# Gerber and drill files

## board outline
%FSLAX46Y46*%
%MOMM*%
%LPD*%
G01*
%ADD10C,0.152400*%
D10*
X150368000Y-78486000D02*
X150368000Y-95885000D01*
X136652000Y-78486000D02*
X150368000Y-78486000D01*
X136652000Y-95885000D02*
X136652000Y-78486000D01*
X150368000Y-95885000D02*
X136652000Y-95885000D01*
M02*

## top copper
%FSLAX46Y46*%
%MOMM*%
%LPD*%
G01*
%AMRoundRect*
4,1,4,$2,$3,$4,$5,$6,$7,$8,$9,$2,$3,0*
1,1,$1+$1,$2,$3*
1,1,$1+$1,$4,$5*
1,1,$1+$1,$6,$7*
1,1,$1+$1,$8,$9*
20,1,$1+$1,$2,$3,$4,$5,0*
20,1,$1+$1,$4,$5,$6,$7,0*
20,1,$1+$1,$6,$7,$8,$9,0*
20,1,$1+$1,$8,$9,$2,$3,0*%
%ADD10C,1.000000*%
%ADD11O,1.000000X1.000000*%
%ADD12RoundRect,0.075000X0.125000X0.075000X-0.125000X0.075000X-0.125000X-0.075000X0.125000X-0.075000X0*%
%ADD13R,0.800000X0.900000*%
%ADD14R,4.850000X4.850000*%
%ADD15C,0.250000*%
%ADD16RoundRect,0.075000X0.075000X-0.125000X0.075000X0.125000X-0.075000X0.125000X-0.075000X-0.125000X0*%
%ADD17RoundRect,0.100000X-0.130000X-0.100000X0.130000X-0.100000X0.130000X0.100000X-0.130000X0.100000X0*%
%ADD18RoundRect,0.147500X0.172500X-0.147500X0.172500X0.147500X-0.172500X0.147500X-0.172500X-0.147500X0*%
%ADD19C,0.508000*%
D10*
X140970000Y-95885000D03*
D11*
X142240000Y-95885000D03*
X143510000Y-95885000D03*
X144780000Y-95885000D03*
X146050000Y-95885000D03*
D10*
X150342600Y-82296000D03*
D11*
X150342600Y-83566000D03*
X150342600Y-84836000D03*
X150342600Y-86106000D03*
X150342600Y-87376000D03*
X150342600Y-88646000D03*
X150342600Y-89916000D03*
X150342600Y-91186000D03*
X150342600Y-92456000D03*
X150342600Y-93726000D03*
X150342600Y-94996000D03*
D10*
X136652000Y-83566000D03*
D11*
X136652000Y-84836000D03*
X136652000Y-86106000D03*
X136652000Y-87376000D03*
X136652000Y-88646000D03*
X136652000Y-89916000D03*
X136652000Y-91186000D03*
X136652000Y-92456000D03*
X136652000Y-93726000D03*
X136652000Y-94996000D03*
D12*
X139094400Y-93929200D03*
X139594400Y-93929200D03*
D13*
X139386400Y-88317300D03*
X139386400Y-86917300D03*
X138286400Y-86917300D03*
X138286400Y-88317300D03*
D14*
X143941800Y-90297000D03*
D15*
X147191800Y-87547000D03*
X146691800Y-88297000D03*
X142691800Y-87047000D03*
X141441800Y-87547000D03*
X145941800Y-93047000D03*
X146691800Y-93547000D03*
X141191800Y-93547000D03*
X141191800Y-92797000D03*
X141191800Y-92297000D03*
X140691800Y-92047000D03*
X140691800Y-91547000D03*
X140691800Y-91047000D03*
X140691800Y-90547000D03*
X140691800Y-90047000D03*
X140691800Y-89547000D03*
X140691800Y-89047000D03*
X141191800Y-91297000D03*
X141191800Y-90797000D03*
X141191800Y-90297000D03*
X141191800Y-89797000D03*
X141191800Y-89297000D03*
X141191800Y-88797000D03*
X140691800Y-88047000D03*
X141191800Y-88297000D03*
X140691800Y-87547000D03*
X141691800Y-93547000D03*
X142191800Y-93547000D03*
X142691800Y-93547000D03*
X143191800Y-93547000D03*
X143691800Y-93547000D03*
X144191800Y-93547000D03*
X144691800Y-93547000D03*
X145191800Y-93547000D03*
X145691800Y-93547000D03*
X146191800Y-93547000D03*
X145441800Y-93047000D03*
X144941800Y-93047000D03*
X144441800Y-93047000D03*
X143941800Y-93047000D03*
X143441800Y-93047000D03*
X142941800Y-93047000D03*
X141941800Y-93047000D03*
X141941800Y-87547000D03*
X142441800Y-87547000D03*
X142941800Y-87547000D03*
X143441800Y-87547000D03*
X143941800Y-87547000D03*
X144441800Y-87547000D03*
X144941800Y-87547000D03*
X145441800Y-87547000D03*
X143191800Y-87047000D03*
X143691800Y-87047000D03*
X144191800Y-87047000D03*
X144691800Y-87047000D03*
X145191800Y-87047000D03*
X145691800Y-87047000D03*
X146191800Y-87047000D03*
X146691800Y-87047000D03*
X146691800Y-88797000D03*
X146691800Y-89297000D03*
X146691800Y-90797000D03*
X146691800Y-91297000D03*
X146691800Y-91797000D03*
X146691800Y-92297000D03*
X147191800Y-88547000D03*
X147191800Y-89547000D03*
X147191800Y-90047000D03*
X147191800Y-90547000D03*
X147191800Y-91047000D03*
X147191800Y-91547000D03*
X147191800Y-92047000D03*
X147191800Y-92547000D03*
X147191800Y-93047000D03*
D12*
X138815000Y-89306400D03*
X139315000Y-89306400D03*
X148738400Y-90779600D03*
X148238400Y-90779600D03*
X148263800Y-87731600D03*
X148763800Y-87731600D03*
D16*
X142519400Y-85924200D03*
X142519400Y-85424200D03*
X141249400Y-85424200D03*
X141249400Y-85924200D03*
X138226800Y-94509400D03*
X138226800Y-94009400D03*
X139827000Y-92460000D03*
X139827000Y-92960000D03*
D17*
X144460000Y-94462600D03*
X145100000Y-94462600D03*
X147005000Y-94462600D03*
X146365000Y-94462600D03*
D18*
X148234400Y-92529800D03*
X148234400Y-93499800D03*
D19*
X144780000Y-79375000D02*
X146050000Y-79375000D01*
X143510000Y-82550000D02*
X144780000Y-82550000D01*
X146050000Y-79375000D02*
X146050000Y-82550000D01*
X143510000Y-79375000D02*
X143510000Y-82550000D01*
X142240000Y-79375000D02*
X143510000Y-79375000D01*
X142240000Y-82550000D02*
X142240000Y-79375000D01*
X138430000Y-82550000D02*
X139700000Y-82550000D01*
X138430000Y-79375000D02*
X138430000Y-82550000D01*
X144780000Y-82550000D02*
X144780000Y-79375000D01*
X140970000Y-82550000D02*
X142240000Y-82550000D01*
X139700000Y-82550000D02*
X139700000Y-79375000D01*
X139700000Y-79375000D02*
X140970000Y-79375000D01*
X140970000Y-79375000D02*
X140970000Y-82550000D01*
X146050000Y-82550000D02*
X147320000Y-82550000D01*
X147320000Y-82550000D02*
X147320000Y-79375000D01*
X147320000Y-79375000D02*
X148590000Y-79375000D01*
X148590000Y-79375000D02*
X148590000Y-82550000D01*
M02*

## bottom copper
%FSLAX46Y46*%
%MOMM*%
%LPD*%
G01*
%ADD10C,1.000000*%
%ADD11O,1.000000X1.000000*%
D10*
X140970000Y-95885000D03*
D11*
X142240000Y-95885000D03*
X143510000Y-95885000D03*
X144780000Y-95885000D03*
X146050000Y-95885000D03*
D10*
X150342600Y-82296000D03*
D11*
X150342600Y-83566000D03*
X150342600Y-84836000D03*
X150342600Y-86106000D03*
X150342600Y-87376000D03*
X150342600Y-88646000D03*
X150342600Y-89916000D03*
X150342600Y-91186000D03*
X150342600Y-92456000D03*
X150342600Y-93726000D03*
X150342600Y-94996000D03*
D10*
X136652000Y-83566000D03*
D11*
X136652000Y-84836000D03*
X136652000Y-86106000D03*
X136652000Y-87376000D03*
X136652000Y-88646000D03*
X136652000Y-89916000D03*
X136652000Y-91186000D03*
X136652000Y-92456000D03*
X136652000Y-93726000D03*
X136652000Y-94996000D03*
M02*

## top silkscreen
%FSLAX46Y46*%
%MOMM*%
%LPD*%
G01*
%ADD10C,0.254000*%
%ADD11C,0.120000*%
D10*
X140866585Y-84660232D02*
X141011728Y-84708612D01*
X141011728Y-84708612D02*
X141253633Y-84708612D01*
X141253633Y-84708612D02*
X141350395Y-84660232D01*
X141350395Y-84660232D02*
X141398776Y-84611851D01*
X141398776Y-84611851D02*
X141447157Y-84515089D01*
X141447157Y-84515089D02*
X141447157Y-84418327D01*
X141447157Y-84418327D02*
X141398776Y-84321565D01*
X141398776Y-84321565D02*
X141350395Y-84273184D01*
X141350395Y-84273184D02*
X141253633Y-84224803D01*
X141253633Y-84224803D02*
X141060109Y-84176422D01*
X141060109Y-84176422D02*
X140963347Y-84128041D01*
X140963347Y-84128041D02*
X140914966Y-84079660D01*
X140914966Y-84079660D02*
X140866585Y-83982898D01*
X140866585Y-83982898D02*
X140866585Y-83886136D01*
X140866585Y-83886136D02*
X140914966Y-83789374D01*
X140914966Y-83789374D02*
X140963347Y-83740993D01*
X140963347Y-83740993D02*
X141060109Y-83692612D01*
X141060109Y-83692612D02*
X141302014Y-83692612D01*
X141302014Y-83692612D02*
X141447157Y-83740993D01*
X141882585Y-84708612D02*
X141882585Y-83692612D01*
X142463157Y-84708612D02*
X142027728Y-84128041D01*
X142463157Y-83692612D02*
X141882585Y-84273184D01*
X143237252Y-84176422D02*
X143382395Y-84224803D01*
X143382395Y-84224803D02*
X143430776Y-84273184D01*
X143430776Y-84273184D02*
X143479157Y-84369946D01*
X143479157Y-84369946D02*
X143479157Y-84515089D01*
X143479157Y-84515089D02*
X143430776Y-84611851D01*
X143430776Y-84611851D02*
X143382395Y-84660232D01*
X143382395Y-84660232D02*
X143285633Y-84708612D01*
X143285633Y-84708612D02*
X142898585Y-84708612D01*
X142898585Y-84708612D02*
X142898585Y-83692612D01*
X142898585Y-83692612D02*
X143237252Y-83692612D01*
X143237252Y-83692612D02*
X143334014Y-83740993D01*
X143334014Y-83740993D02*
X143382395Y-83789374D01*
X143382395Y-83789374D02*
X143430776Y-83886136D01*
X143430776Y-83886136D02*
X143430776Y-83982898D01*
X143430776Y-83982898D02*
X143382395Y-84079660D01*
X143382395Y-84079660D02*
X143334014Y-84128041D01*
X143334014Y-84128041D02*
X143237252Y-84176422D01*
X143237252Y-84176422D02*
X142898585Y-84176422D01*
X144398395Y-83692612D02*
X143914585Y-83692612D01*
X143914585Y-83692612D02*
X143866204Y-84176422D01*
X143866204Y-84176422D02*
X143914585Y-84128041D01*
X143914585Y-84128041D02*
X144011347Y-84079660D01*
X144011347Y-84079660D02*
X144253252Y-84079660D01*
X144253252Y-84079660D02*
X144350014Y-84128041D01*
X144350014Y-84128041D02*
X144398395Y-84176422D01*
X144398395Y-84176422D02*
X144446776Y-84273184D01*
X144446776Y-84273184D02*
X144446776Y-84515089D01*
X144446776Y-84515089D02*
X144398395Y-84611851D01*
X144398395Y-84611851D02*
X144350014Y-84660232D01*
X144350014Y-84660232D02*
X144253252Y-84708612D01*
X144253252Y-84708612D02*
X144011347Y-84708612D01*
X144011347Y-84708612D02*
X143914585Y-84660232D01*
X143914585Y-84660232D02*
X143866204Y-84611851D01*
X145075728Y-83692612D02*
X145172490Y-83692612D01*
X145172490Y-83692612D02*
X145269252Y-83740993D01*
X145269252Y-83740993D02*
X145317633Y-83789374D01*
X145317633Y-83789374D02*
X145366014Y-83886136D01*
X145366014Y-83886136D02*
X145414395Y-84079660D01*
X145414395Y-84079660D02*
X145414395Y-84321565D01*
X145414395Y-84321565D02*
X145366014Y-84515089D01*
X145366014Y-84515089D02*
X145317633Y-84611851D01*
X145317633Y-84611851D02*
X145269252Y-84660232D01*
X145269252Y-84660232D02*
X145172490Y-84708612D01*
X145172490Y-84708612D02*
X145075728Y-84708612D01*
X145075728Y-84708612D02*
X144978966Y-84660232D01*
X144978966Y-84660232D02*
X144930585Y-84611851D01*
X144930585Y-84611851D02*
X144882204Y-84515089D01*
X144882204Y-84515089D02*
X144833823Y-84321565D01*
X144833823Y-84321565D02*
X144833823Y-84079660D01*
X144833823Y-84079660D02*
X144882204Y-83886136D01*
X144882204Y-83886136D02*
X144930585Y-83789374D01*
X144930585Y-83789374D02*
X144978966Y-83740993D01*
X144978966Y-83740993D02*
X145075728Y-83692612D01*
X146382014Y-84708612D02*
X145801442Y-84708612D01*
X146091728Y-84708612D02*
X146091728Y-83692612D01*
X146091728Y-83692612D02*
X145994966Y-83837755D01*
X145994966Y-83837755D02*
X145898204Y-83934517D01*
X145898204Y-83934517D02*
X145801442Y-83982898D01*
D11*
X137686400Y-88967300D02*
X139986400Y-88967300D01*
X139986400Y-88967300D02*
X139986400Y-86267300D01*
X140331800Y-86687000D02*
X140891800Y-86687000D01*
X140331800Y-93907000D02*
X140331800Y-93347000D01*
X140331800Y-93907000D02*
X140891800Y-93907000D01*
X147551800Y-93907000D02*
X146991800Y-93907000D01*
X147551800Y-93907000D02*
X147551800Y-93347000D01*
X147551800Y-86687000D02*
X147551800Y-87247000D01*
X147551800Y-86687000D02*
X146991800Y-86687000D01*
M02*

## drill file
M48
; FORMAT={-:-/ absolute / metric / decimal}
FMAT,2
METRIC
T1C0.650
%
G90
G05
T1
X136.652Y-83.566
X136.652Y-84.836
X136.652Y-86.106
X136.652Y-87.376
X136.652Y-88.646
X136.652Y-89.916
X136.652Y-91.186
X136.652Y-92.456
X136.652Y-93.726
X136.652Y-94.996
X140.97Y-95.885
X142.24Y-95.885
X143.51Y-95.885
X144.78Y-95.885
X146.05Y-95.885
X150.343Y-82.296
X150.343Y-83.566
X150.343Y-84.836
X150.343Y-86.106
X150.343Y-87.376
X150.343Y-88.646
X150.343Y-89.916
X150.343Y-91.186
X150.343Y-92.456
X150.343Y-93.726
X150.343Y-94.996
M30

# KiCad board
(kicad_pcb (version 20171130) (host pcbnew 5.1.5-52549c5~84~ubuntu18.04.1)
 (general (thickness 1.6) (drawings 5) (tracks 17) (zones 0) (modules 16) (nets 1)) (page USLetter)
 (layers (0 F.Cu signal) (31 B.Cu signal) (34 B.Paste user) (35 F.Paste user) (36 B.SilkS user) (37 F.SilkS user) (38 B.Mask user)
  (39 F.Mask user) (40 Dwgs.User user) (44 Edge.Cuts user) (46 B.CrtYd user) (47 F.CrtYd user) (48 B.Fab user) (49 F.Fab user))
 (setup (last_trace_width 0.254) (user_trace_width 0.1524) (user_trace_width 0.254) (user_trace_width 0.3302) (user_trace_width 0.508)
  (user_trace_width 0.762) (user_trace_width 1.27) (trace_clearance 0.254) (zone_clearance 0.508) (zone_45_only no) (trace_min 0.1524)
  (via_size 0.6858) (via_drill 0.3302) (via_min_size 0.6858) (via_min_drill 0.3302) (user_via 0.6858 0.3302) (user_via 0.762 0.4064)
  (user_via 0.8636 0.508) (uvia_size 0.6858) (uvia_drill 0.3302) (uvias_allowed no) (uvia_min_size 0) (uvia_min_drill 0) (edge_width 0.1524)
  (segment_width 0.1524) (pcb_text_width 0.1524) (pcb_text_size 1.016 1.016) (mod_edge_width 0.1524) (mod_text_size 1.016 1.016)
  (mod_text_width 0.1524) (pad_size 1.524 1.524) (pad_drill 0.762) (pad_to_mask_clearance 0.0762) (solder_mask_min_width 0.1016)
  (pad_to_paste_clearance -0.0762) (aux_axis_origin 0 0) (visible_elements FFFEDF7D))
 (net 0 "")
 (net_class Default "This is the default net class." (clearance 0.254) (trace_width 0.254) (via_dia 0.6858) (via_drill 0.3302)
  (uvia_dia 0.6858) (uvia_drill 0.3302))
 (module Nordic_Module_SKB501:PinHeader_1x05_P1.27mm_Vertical (layer F.Cu) (at 140.97 95.885 90)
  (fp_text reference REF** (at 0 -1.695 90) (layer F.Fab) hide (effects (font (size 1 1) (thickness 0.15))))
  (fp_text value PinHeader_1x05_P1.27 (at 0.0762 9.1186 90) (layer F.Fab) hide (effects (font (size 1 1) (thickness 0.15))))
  (pad 1 thru_hole circle (at 0 0 90) (size 1 1) (drill 0.65) (layers *.Cu *.Mask))
  (pad 2 thru_hole oval (at 0 1.27 90) (size 1 1) (drill 0.65) (layers *.Cu *.Mask))
  (pad 3 thru_hole oval (at 0 2.54 90) (size 1 1) (drill 0.65) (layers *.Cu *.Mask))
  (pad 4 thru_hole oval (at 0 3.81 90) (size 1 1) (drill 0.65) (layers *.Cu *.Mask))
  (pad 5 thru_hole oval (at 0 5.08 90) (size 1 1) (drill 0.65) (layers *.Cu *.Mask)))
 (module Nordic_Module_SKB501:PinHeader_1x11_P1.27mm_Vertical (layer F.Cu) (at 150.3426 82.296)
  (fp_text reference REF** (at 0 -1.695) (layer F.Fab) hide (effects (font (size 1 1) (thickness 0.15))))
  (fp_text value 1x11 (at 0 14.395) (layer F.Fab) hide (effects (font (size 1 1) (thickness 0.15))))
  (pad 1 thru_hole circle (at 0 0) (size 1 1) (drill 0.65) (layers *.Cu *.Mask))
  (pad 2 thru_hole oval (at 0 1.27) (size 1 1) (drill 0.65) (layers *.Cu *.Mask))
  (pad 3 thru_hole oval (at 0 2.54) (size 1 1) (drill 0.65) (layers *.Cu *.Mask))
  (pad 4 thru_hole oval (at 0 3.81) (size 1 1) (drill 0.65) (layers *.Cu *.Mask))
  (pad 5 thru_hole oval (at 0 5.08) (size 1 1) (drill 0.65) (layers *.Cu *.Mask))
  (pad 6 thru_hole oval (at 0 6.35) (size 1 1) (drill 0.65) (layers *.Cu *.Mask))
  (pad 7 thru_hole oval (at 0 7.62) (size 1 1) (drill 0.65) (layers *.Cu *.Mask))
  (pad 8 thru_hole oval (at 0 8.89) (size 1 1) (drill 0.65) (layers *.Cu *.Mask))
  (pad 9 thru_hole oval (at 0 10.16) (size 1 1) (drill 0.65) (layers *.Cu *.Mask))
  (pad 10 thru_hole oval (at 0 11.43) (size 1 1) (drill 0.65) (layers *.Cu *.Mask))
  (pad 11 thru_hole oval (at 0 12.7) (size 1 1) (drill 0.65) (layers *.Cu *.Mask)))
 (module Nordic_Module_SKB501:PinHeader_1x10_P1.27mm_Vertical (layer F.Cu) (at 136.652 83.566)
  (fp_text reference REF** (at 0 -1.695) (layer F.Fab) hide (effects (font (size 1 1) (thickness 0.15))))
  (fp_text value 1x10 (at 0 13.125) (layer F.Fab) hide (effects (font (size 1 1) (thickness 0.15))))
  (pad 1 thru_hole circle (at 0 0) (size 1 1) (drill 0.65) (layers *.Cu *.Mask))
  (pad 2 thru_hole oval (at 0 1.27) (size 1 1) (drill 0.65) (layers *.Cu *.Mask))
  (pad 3 thru_hole oval (at 0 2.54) (size 1 1) (drill 0.65) (layers *.Cu *.Mask))
  (pad 4 thru_hole oval (at 0 3.81) (size 1 1) (drill 0.65) (layers *.Cu *.Mask))
  (pad 5 thru_hole oval (at 0 5.08) (size 1 1) (drill 0.65) (layers *.Cu *.Mask))
  (pad 6 thru_hole oval (at 0 6.35) (size 1 1) (drill 0.65) (layers *.Cu *.Mask))
  (pad 7 thru_hole oval (at 0 7.62) (size 1 1) (drill 0.65) (layers *.Cu *.Mask))
  (pad 8 thru_hole oval (at 0 8.89) (size 1 1) (drill 0.65) (layers *.Cu *.Mask))
  (pad 9 thru_hole oval (at 0 10.16) (size 1 1) (drill 0.65) (layers *.Cu *.Mask))
  (pad 10 thru_hole oval (at 0 11.43) (size 1 1) (drill 0.65) (layers *.Cu *.Mask)))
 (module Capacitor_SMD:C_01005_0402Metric (layer F.Cu) (at 139.3444 93.9292 180)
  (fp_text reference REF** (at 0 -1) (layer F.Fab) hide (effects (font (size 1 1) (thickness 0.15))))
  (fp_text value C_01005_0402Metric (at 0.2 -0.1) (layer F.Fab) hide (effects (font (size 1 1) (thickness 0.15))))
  (pad 2 smd roundrect (at 0.25 0 180) (size 0.4 0.3) (layers F.Cu F.Mask) (roundrect_rratio 0.25))
  (pad 1 smd roundrect (at -0.25 0 180) (size 0.4 0.3) (layers F.Cu F.Mask) (roundrect_rratio 0.25))
  (pad "" smd roundrect (at 0.275 0 180) (size 0.27 0.27) (layers F.Paste) (roundrect_rratio 0.25))
  (pad "" smd roundrect (at -0.275 0 180) (size 0.27 0.27) (layers F.Paste) (roundrect_rratio 0.25)))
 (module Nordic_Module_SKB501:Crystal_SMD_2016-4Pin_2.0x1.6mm (layer F.Cu) (at 138.8364 87.6173 90)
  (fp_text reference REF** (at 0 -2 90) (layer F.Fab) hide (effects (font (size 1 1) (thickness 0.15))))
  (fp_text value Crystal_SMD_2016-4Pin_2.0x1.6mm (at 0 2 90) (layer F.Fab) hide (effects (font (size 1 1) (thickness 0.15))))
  (fp_line (start -1.35 -1.15) (end -1.35 1.15) (layer F.SilkS) (width 0.12))
  (fp_line (start -1.35 1.15) (end 1.35 1.15) (layer F.SilkS) (width 0.12))
  (pad 1 smd rect (at -0.7 0.55 90) (size 0.9 0.8) (layers F.Cu F.Paste F.Mask))
  (pad 2 smd rect (at 0.7 0.55 90) (size 0.9 0.8) (layers F.Cu F.Paste F.Mask))
  (pad 3 smd rect (at 0.7 -0.55 90) (size 0.9 0.8) (layers F.Cu F.Paste F.Mask))
  (pad 4 smd rect (at -0.7 -0.55 90) (size 0.9 0.8) (layers F.Cu F.Paste F.Mask)))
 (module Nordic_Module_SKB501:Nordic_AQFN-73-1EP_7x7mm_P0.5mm (layer F.Cu) (at 143.9418 90.297)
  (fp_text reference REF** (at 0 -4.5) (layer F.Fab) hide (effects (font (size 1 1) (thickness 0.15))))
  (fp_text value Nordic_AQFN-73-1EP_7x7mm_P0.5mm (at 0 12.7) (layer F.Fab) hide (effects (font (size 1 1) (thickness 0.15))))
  (fp_line (start -3.61 -3.61) (end -3.05 -3.61) (layer F.SilkS) (width 0.12))
  (fp_line (start -3.61 3.61) (end -3.61 3.05) (layer F.SilkS) (width 0.12))
  (fp_line (start -3.61 3.61) (end -3.05 3.61) (layer F.SilkS) (width 0.12))
  (fp_line (start 3.61 3.61) (end 3.05 3.61) (layer F.SilkS) (width 0.12))
  (fp_line (start 3.61 3.61) (end 3.61 3.05) (layer F.SilkS) (width 0.12))
  (fp_line (start 3.61 -3.61) (end 3.61 -3.05) (layer F.SilkS) (width 0.12))
  (fp_line (start 3.61 -3.61) (end 3.05 -3.61) (layer F.SilkS) (width 0.12))
  (pad "" smd rect (at 1.2125 1.2125 180) (size 2 2) (layers F.Paste))
  (pad "" smd rect (at -1.2125 1.2125 180) (size 2 2) (layers F.Paste))
  (pad "" smd rect (at 1.2125 -1.2125 180) (size 2 2) (layers F.Paste))
  (pad "" smd rect (at -1.2125 -1.2125 180) (size 2 2) (layers F.Paste))
  (pad EP smd rect (at 0 0 180) (size 4.85 4.85) (layers F.Cu F.Mask))
  (pad B24 smd circle (at 3.25 -2.75 180) (size 0.25 0.25) (layers F.Cu F.Paste F.Mask))
  (pad D23 smd circle (at 2.75 -2 180) (size 0.25 0.25) (layers F.Cu F.Paste F.Mask))
  (pad A8 smd circle (at -1.25 -3.25 180) (size 0.25 0.25) (layers F.Cu F.Paste F.Mask))
  (pad B3 smd circle (at -2.5 -2.75 180) (size 0.25 0.25) (layers F.Cu F.Paste F.Mask))
  (pad AC21 smd circle (at 2 2.75 180) (size 0.25 0.25) (layers F.Cu F.Paste F.Mask))
  (pad AD23 smd circle (at 2.75 3.25 180) (size 0.25 0.25) (layers F.Cu F.Paste F.Mask))
  (pad AD2 smd circle (at -2.75 3.25 180) (size 0.25 0.25) (layers F.Cu F.Paste F.Mask))
  (pad AB2 smd circle (at -2.75 2.5 180) (size 0.25 0.25) (layers F.Cu F.Paste F.Mask))
  (pad Y2 smd circle (at -2.75 2 180) (size 0.25 0.25) (layers F.Cu F.Paste F.Mask))
  (pad W1 smd circle (at -3.25 1.75 180) (size 0.25 0.25) (layers F.Cu F.Paste F.Mask))
  (pad U1 smd circle (at -3.25 1.25 180) (size 0.25 0.25) (layers F.Cu F.Paste F.Mask))
  (pad R1 smd circle (at -3.25 0.75 180) (size 0.25 0.25) (layers F.Cu F.Paste F.Mask))
  (pad N1 smd circle (at -3.25 0.25 180) (size 0.25 0.25) (layers F.Cu F.Paste F.Mask))
  (pad L1 smd circle (at -3.25 -0.25 180) (size 0.25 0.25) (layers F.Cu F.Paste F.Mask))
  (pad J1 smd circle (at -3.25 -0.75 180) (size 0.25 0.25) (layers F.Cu F.Paste F.Mask))
  (pad G1 smd circle (at -3.25 -1.25 180) (size 0.25 0.25) (layers F.Cu F.Paste F.Mask))
  (pad T2 smd circle (at -2.75 1 180) (size 0.25 0.25) (layers F.Cu F.Paste F.Mask))
  (pad P2 smd circle (at -2.75 0.5 180) (size 0.25 0.25) (layers F.Cu F.Paste F.Mask))
  (pad M2 smd circle (at -2.75 0 180) (size 0.25 0.25) (layers F.Cu F.Paste F.Mask))
  (pad K2 smd circle (at -2.75 -0.5 180) (size 0.25 0.25) (layers F.Cu F.Paste F.Mask))
  (pad H2 smd circle (at -2.75 -1 180) (size 0.25 0.25) (layers F.Cu F.Paste F.Mask))
  (pad F2 smd circle (at -2.75 -1.5 180) (size 0.25 0.25) (layers F.Cu F.Paste F.Mask))
  (pad C1 smd circle (at -3.25 -2.25 180) (size 0.25 0.25) (layers F.Cu F.Paste F.Mask))
  (pad D2 smd circle (at -2.75 -2 180) (size 0.25 0.25) (layers F.Cu F.Paste F.Mask))
  (pad B1 smd circle (at -3.25 -2.75 180) (size 0.25 0.25) (layers F.Cu F.Paste F.Mask))
  (pad AD4 smd circle (at -2.25 3.25 180) (size 0.25 0.25) (layers F.Cu F.Paste F.Mask))
  (pad AD6 smd circle (at -1.75 3.25 180) (size 0.25 0.25) (layers F.Cu F.Paste F.Mask))
  (pad AD8 smd circle (at -1.25 3.25 180) (size 0.25 0.25) (layers F.Cu F.Paste F.Mask))
  (pad AD10 smd circle (at -0.75 3.25 180) (size 0.25 0.25) (layers F.Cu F.Paste F.Mask))
  (pad AD12 smd circle (at -0.25 3.25 180) (size 0.25 0.25) (layers F.Cu F.Paste F.Mask))
  (pad AD14 smd circle (at 0.25 3.25 180) (size 0.25 0.25) (layers F.Cu F.Paste F.Mask))
  (pad AD16 smd circle (at 0.75 3.25 180) (size 0.25 0.25) (layers F.Cu F.Paste F.Mask))
  (pad AD18 smd circle (at 1.25 3.25 180) (size 0.25 0.25) (layers F.Cu F.Paste F.Mask))
  (pad AD20 smd circle (at 1.75 3.25 180) (size 0.25 0.25) (layers F.Cu F.Paste F.Mask))
  (pad AD22 smd circle (at 2.25 3.25 180) (size 0.25 0.25) (layers F.Cu F.Paste F.Mask))
  (pad AC19 smd circle (at 1.5 2.75 180) (size 0.25 0.25) (layers F.Cu F.Paste F.Mask))
  (pad AC17 smd circle (at 1 2.75 180) (size 0.25 0.25) (layers F.Cu F.Paste F.Mask))
  (pad AC15 smd circle (at 0.5 2.75 180) (size 0.25 0.25) (layers F.Cu F.Paste F.Mask))
  (pad AC13 smd circle (at 0 2.75 180) (size 0.25 0.25) (layers F.Cu F.Paste F.Mask))
  (pad AC11 smd circle (at -0.5 2.75 180) (size 0.25 0.25) (layers F.Cu F.Paste F.Mask))
  (pad AC9 smd circle (at -1 2.75 180) (size 0.25 0.25) (layers F.Cu F.Paste F.Mask))
  (pad AC5 smd circle (at -2 2.75 180) (size 0.25 0.25) (layers F.Cu F.Paste F.Mask))
  (pad B5 smd circle (at -2 -2.75 180) (size 0.25 0.25) (layers F.Cu F.Paste F.Mask))
  (pad B7 smd circle (at -1.5 -2.75 180) (size 0.25 0.25) (layers F.Cu F.Paste F.Mask))
  (pad B9 smd circle (at -1 -2.75 180) (size 0.25 0.25) (layers F.Cu F.Paste F.Mask))
  (pad B11 smd circle (at -0.5 -2.75 180) (size 0.25 0.25) (layers F.Cu F.Paste F.Mask))
  (pad B13 smd circle (at 0 -2.75 180) (size 0.25 0.25) (layers F.Cu F.Paste F.Mask))
  (pad B15 smd circle (at 0.5 -2.75 180) (size 0.25 0.25) (layers F.Cu F.Paste F.Mask))
  (pad B17 smd circle (at 1 -2.75 180) (size 0.25 0.25) (layers F.Cu F.Paste F.Mask))
  (pad B19 smd circle (at 1.5 -2.75 180) (size 0.25 0.25) (layers F.Cu F.Paste F.Mask))
  (pad A10 smd circle (at -0.75 -3.25 180) (size 0.25 0.25) (layers F.Cu F.Paste F.Mask))
  (pad A12 smd circle (at -0.25 -3.25 180) (size 0.25 0.25) (layers F.Cu F.Paste F.Mask))
  (pad A14 smd circle (at 0.25 -3.25 180) (size 0.25 0.25) (layers F.Cu F.Paste F.Mask))
  (pad A16 smd circle (at 0.75 -3.25 180) (size 0.25 0.25) (layers F.Cu F.Paste F.Mask))
  (pad A18 smd circle (at 1.25 -3.25 180) (size 0.25 0.25) (layers F.Cu F.Paste F.Mask))
  (pad A20 smd circle (at 1.75 -3.25 180) (size 0.25 0.25) (layers F.Cu F.Paste F.Mask))
  (pad A22 smd circle (at 2.25 -3.25 180) (size 0.25 0.25) (layers F.Cu F.Paste F.Mask))
  (pad A23 smd circle (at 2.75 -3.25 180) (size 0.25 0.25) (layers F.Cu F.Paste F.Mask))
  (pad F23 smd circle (at 2.75 -1.5 180) (size 0.25 0.25) (layers F.Cu F.Paste F.Mask))
  (pad H23 smd circle (at 2.75 -1 180) (size 0.25 0.25) (layers F.Cu F.Paste F.Mask))
  (pad P23 smd circle (at 2.75 0.5 180) (size 0.25 0.25) (layers F.Cu F.Paste F.Mask))
  (pad T23 smd circle (at 2.75 1 180) (size 0.25 0.25) (layers F.Cu F.Paste F.Mask))
  (pad V23 smd circle (at 2.75 1.5 180) (size 0.25 0.25) (layers F.Cu F.Paste F.Mask))
  (pad Y23 smd circle (at 2.75 2 180) (size 0.25 0.25) (layers F.Cu F.Paste F.Mask))
  (pad E24 smd circle (at 3.25 -1.75 180) (size 0.25 0.25) (layers F.Cu F.Paste F.Mask))
  (pad J24 smd circle (at 3.25 -0.75 180) (size 0.25 0.25) (layers F.Cu F.Paste F.Mask))
  (pad L24 smd circle (at 3.25 -0.25 180) (size 0.25 0.25) (layers F.Cu F.Paste F.Mask))
  (pad N24 smd circle (at 3.25 0.25 180) (size 0.25 0.25) (layers F.Cu F.Paste F.Mask))
  (pad R24 smd circle (at 3.25 0.75 180) (size 0.25 0.25) (layers F.Cu F.Paste F.Mask))
  (pad U24 smd circle (at 3.25 1.25 180) (size 0.25 0.25) (layers F.Cu F.Paste F.Mask))
  (pad W24 smd circle (at 3.25 1.75 180) (size 0.25 0.25) (layers F.Cu F.Paste F.Mask))
  (pad AA24 smd circle (at 3.25 2.25 180) (size 0.25 0.25) (layers F.Cu F.Paste F.Mask))
  (pad AC24 smd circle (at 3.25 2.75 180) (size 0.25 0.25) (layers F.Cu F.Paste F.Mask)))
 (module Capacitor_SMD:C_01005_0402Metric (layer F.Cu) (at 139.065 89.3064 180)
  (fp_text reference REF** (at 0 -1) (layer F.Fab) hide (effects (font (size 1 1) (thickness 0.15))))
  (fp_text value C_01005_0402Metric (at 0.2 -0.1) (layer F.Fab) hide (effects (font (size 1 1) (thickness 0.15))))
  (pad 2 smd roundrect (at 0.25 0 180) (size 0.4 0.3) (layers F.Cu F.Mask) (roundrect_rratio 0.25))
  (pad 1 smd roundrect (at -0.25 0 180) (size 0.4 0.3) (layers F.Cu F.Mask) (roundrect_rratio 0.25))
  (pad "" smd roundrect (at 0.275 0 180) (size 0.27 0.27) (layers F.Paste) (roundrect_rratio 0.25))
  (pad "" smd roundrect (at -0.275 0 180) (size 0.27 0.27) (layers F.Paste) (roundrect_rratio 0.25)))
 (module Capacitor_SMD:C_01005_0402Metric (layer F.Cu) (at 148.4884 90.7796 180)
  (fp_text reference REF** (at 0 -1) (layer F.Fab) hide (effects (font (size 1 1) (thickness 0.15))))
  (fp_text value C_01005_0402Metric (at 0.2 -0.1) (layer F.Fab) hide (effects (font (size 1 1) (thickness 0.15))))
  (pad "" smd roundrect (at -0.275 0 180) (size 0.27 0.27) (layers F.Paste) (roundrect_rratio 0.25))
  (pad "" smd roundrect (at 0.275 0 180) (size 0.27 0.27) (layers F.Paste) (roundrect_rratio 0.25))
  (pad 1 smd roundrect (at -0.25 0 180) (size 0.4 0.3) (layers F.Cu F.Mask) (roundrect_rratio 0.25))
  (pad 2 smd roundrect (at 0.25 0 180) (size 0.4 0.3) (layers F.Cu F.Mask) (roundrect_rratio 0.25)))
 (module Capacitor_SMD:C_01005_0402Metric (layer F.Cu) (at 148.5138 87.7316 180)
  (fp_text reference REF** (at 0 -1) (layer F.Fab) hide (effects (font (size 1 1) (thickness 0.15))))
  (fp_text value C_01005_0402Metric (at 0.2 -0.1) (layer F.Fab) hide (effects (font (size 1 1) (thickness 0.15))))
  (pad 2 smd roundrect (at 0.25 0 180) (size 0.4 0.3) (layers F.Cu F.Mask) (roundrect_rratio 0.25))
  (pad 1 smd roundrect (at -0.25 0 180) (size 0.4 0.3) (layers F.Cu F.Mask) (roundrect_rratio 0.25))
  (pad "" smd roundrect (at 0.275 0 180) (size 0.27 0.27) (layers F.Paste) (roundrect_rratio 0.25))
  (pad "" smd roundrect (at -0.275 0 180) (size 0.27 0.27) (layers F.Paste) (roundrect_rratio 0.25)))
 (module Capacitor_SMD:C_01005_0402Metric (layer F.Cu) (at 142.5194 85.6742 90)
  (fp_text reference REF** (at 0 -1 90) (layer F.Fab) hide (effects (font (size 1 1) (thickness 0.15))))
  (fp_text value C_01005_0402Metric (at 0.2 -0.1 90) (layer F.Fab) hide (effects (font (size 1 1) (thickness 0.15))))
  (pad "" smd roundrect (at -0.275 0 90) (size 0.27 0.27) (layers F.Paste) (roundrect_rratio 0.25))
  (pad "" smd roundrect (at 0.275 0 90) (size 0.27 0.27) (layers F.Paste) (roundrect_rratio 0.25))
  (pad 1 smd roundrect (at -0.25 0 90) (size 0.4 0.3) (layers F.Cu F.Mask) (roundrect_rratio 0.25))
  (pad 2 smd roundrect (at 0.25 0 90) (size 0.4 0.3) (layers F.Cu F.Mask) (roundrect_rratio 0.25)))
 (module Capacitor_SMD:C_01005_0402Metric (layer F.Cu) (at 141.2494 85.6742 90)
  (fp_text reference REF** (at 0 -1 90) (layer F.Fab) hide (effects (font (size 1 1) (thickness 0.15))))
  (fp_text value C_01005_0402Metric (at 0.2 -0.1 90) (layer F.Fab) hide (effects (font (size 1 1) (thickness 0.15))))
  (pad 2 smd roundrect (at 0.25 0 90) (size 0.4 0.3) (layers F.Cu F.Mask) (roundrect_rratio 0.25))
  (pad 1 smd roundrect (at -0.25 0 90) (size 0.4 0.3) (layers F.Cu F.Mask) (roundrect_rratio 0.25))
  (pad "" smd roundrect (at 0.275 0 90) (size 0.27 0.27) (layers F.Paste) (roundrect_rratio 0.25))
  (pad "" smd roundrect (at -0.275 0 90) (size 0.27 0.27) (layers F.Paste) (roundrect_rratio 0.25)))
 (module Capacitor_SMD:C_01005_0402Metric (layer F.Cu) (at 138.2268 94.2594 90)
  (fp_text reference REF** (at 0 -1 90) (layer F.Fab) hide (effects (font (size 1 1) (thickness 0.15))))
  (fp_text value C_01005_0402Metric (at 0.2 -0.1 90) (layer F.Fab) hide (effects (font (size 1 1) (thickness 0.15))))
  (pad "" smd roundrect (at -0.275 0 90) (size 0.27 0.27) (layers F.Paste) (roundrect_rratio 0.25))
  (pad "" smd roundrect (at 0.275 0 90) (size 0.27 0.27) (layers F.Paste) (roundrect_rratio 0.25))
  (pad 1 smd roundrect (at -0.25 0 90) (size 0.4 0.3) (layers F.Cu F.Mask) (roundrect_rratio 0.25))
  (pad 2 smd roundrect (at 0.25 0 90) (size 0.4 0.3) (layers F.Cu F.Mask) (roundrect_rratio 0.25)))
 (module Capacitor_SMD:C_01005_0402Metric (layer F.Cu) (at 139.827 92.71 90)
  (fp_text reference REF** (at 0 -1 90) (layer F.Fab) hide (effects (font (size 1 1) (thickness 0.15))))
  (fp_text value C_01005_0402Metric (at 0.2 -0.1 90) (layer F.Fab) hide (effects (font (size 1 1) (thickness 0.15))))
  (pad 2 smd roundrect (at 0.25 0 90) (size 0.4 0.3) (layers F.Cu F.Mask) (roundrect_rratio 0.25))
  (pad 1 smd roundrect (at -0.25 0 90) (size 0.4 0.3) (layers F.Cu F.Mask) (roundrect_rratio 0.25))
  (pad "" smd roundrect (at 0.275 0 90) (size 0.27 0.27) (layers F.Paste) (roundrect_rratio 0.25))
  (pad "" smd roundrect (at -0.275 0 90) (size 0.27 0.27) (layers F.Paste) (roundrect_rratio 0.25)))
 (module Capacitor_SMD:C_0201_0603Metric (layer F.Cu) (at 144.78 94.4626)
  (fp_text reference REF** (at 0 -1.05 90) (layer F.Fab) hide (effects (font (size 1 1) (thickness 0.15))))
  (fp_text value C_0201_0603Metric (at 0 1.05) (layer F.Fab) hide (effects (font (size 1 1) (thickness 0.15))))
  (pad "" smd roundrect (at -0.345 0) (size 0.318 0.36) (layers F.Paste) (roundrect_rratio 0.25))
  (pad "" smd roundrect (at 0.345 0) (size 0.318 0.36) (layers F.Paste) (roundrect_rratio 0.25))
  (pad 1 smd roundrect (at -0.32 0) (size 0.46 0.4) (layers F.Cu F.Mask) (roundrect_rratio 0.25))
  (pad 2 smd roundrect (at 0.32 0) (size 0.46 0.4) (layers F.Cu F.Mask) (roundrect_rratio 0.25)))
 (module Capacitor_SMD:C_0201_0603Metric (layer F.Cu) (at 146.685 94.4626)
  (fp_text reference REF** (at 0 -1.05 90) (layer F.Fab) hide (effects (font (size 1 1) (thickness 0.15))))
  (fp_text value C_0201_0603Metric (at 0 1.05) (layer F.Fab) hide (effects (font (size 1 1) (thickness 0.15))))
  (pad 2 smd roundrect (at 0.32 0) (size 0.46 0.4) (layers F.Cu F.Mask) (roundrect_rratio 0.25))
  (pad 1 smd roundrect (at -0.32 0) (size 0.46 0.4) (layers F.Cu F.Mask) (roundrect_rratio 0.25))
  (pad "" smd roundrect (at 0.345 0) (size 0.318 0.36) (layers F.Paste) (roundrect_rratio 0.25))
  (pad "" smd roundrect (at -0.345 0) (size 0.318 0.36) (layers F.Paste) (roundrect_rratio 0.25)))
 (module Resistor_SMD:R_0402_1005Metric (layer F.Cu) (at 148.2344 93.0148 90)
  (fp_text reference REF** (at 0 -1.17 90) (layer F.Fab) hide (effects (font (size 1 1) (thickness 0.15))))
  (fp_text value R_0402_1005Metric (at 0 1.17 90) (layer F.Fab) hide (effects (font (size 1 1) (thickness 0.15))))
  (pad 2 smd roundrect (at 0.485 0 90) (size 0.59 0.64) (layers F.Cu F.Paste F.Mask) (roundrect_rratio 0.25))
  (pad 1 smd roundrect (at -0.485 0 90) (size 0.59 0.64) (layers F.Cu F.Paste F.Mask) (roundrect_rratio 0.25)))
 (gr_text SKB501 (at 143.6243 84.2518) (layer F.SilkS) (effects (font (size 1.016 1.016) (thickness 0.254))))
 (gr_line (start 150.368 78.486) (end 150.368 95.885) (layer Edge.Cuts) (width 0.1524))
 (gr_line (start 136.652 78.486) (end 150.368 78.486) (layer Edge.Cuts) (width 0.1524))
 (gr_line (start 136.652 95.885) (end 136.652 78.486) (layer Edge.Cuts) (width 0.1524))
 (gr_line (start 150.368 95.885) (end 136.652 95.885) (layer Edge.Cuts) (width 0.1524))
 (segment (start 144.78 79.375) (end 146.05 79.375) (width 0.508) (layer F.Cu) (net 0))
 (segment (start 143.51 82.55) (end 144.78 82.55) (width 0.508) (layer F.Cu) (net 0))
 (segment (start 146.05 79.375) (end 146.05 82.55) (width 0.508) (layer F.Cu) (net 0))
 (segment (start 143.51 79.375) (end 143.51 82.55) (width 0.508) (layer F.Cu) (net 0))
 (segment (start 142.24 79.375) (end 143.51 79.375) (width 0.508) (layer F.Cu) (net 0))
 (segment (start 142.24 82.55) (end 142.24 79.375) (width 0.508) (layer F.Cu) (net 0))
 (segment (start 138.43 82.55) (end 139.7 82.55) (width 0.508) (layer F.Cu) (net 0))
 (segment (start 138.43 79.375) (end 138.43 82.55) (width 0.508) (layer F.Cu) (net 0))
 (segment (start 144.78 82.55) (end 144.78 79.375) (width 0.508) (layer F.Cu) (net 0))
 (segment (start 140.97 82.55) (end 142.24 82.55) (width 0.508) (layer F.Cu) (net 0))
 (segment (start 139.7 82.55) (end 139.7 79.375) (width 0.508) (layer F.Cu) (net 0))
 (segment (start 139.7 79.375) (end 140.97 79.375) (width 0.508) (layer F.Cu) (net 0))
 (segment (start 140.97 79.375) (end 140.97 82.55) (width 0.508) (layer F.Cu) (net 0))
 (segment (start 146.05 82.55) (end 147.32 82.55) (width 0.508) (layer F.Cu) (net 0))
 (segment (start 147.32 82.55) (end 147.32 79.375) (width 0.508) (layer F.Cu) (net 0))
 (segment (start 147.32 79.375) (end 148.59 79.375) (width 0.508) (layer F.Cu) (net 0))
 (segment (start 148.59 79.375) (end 148.59 82.55) (width 0.508) (layer F.Cu) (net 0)))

